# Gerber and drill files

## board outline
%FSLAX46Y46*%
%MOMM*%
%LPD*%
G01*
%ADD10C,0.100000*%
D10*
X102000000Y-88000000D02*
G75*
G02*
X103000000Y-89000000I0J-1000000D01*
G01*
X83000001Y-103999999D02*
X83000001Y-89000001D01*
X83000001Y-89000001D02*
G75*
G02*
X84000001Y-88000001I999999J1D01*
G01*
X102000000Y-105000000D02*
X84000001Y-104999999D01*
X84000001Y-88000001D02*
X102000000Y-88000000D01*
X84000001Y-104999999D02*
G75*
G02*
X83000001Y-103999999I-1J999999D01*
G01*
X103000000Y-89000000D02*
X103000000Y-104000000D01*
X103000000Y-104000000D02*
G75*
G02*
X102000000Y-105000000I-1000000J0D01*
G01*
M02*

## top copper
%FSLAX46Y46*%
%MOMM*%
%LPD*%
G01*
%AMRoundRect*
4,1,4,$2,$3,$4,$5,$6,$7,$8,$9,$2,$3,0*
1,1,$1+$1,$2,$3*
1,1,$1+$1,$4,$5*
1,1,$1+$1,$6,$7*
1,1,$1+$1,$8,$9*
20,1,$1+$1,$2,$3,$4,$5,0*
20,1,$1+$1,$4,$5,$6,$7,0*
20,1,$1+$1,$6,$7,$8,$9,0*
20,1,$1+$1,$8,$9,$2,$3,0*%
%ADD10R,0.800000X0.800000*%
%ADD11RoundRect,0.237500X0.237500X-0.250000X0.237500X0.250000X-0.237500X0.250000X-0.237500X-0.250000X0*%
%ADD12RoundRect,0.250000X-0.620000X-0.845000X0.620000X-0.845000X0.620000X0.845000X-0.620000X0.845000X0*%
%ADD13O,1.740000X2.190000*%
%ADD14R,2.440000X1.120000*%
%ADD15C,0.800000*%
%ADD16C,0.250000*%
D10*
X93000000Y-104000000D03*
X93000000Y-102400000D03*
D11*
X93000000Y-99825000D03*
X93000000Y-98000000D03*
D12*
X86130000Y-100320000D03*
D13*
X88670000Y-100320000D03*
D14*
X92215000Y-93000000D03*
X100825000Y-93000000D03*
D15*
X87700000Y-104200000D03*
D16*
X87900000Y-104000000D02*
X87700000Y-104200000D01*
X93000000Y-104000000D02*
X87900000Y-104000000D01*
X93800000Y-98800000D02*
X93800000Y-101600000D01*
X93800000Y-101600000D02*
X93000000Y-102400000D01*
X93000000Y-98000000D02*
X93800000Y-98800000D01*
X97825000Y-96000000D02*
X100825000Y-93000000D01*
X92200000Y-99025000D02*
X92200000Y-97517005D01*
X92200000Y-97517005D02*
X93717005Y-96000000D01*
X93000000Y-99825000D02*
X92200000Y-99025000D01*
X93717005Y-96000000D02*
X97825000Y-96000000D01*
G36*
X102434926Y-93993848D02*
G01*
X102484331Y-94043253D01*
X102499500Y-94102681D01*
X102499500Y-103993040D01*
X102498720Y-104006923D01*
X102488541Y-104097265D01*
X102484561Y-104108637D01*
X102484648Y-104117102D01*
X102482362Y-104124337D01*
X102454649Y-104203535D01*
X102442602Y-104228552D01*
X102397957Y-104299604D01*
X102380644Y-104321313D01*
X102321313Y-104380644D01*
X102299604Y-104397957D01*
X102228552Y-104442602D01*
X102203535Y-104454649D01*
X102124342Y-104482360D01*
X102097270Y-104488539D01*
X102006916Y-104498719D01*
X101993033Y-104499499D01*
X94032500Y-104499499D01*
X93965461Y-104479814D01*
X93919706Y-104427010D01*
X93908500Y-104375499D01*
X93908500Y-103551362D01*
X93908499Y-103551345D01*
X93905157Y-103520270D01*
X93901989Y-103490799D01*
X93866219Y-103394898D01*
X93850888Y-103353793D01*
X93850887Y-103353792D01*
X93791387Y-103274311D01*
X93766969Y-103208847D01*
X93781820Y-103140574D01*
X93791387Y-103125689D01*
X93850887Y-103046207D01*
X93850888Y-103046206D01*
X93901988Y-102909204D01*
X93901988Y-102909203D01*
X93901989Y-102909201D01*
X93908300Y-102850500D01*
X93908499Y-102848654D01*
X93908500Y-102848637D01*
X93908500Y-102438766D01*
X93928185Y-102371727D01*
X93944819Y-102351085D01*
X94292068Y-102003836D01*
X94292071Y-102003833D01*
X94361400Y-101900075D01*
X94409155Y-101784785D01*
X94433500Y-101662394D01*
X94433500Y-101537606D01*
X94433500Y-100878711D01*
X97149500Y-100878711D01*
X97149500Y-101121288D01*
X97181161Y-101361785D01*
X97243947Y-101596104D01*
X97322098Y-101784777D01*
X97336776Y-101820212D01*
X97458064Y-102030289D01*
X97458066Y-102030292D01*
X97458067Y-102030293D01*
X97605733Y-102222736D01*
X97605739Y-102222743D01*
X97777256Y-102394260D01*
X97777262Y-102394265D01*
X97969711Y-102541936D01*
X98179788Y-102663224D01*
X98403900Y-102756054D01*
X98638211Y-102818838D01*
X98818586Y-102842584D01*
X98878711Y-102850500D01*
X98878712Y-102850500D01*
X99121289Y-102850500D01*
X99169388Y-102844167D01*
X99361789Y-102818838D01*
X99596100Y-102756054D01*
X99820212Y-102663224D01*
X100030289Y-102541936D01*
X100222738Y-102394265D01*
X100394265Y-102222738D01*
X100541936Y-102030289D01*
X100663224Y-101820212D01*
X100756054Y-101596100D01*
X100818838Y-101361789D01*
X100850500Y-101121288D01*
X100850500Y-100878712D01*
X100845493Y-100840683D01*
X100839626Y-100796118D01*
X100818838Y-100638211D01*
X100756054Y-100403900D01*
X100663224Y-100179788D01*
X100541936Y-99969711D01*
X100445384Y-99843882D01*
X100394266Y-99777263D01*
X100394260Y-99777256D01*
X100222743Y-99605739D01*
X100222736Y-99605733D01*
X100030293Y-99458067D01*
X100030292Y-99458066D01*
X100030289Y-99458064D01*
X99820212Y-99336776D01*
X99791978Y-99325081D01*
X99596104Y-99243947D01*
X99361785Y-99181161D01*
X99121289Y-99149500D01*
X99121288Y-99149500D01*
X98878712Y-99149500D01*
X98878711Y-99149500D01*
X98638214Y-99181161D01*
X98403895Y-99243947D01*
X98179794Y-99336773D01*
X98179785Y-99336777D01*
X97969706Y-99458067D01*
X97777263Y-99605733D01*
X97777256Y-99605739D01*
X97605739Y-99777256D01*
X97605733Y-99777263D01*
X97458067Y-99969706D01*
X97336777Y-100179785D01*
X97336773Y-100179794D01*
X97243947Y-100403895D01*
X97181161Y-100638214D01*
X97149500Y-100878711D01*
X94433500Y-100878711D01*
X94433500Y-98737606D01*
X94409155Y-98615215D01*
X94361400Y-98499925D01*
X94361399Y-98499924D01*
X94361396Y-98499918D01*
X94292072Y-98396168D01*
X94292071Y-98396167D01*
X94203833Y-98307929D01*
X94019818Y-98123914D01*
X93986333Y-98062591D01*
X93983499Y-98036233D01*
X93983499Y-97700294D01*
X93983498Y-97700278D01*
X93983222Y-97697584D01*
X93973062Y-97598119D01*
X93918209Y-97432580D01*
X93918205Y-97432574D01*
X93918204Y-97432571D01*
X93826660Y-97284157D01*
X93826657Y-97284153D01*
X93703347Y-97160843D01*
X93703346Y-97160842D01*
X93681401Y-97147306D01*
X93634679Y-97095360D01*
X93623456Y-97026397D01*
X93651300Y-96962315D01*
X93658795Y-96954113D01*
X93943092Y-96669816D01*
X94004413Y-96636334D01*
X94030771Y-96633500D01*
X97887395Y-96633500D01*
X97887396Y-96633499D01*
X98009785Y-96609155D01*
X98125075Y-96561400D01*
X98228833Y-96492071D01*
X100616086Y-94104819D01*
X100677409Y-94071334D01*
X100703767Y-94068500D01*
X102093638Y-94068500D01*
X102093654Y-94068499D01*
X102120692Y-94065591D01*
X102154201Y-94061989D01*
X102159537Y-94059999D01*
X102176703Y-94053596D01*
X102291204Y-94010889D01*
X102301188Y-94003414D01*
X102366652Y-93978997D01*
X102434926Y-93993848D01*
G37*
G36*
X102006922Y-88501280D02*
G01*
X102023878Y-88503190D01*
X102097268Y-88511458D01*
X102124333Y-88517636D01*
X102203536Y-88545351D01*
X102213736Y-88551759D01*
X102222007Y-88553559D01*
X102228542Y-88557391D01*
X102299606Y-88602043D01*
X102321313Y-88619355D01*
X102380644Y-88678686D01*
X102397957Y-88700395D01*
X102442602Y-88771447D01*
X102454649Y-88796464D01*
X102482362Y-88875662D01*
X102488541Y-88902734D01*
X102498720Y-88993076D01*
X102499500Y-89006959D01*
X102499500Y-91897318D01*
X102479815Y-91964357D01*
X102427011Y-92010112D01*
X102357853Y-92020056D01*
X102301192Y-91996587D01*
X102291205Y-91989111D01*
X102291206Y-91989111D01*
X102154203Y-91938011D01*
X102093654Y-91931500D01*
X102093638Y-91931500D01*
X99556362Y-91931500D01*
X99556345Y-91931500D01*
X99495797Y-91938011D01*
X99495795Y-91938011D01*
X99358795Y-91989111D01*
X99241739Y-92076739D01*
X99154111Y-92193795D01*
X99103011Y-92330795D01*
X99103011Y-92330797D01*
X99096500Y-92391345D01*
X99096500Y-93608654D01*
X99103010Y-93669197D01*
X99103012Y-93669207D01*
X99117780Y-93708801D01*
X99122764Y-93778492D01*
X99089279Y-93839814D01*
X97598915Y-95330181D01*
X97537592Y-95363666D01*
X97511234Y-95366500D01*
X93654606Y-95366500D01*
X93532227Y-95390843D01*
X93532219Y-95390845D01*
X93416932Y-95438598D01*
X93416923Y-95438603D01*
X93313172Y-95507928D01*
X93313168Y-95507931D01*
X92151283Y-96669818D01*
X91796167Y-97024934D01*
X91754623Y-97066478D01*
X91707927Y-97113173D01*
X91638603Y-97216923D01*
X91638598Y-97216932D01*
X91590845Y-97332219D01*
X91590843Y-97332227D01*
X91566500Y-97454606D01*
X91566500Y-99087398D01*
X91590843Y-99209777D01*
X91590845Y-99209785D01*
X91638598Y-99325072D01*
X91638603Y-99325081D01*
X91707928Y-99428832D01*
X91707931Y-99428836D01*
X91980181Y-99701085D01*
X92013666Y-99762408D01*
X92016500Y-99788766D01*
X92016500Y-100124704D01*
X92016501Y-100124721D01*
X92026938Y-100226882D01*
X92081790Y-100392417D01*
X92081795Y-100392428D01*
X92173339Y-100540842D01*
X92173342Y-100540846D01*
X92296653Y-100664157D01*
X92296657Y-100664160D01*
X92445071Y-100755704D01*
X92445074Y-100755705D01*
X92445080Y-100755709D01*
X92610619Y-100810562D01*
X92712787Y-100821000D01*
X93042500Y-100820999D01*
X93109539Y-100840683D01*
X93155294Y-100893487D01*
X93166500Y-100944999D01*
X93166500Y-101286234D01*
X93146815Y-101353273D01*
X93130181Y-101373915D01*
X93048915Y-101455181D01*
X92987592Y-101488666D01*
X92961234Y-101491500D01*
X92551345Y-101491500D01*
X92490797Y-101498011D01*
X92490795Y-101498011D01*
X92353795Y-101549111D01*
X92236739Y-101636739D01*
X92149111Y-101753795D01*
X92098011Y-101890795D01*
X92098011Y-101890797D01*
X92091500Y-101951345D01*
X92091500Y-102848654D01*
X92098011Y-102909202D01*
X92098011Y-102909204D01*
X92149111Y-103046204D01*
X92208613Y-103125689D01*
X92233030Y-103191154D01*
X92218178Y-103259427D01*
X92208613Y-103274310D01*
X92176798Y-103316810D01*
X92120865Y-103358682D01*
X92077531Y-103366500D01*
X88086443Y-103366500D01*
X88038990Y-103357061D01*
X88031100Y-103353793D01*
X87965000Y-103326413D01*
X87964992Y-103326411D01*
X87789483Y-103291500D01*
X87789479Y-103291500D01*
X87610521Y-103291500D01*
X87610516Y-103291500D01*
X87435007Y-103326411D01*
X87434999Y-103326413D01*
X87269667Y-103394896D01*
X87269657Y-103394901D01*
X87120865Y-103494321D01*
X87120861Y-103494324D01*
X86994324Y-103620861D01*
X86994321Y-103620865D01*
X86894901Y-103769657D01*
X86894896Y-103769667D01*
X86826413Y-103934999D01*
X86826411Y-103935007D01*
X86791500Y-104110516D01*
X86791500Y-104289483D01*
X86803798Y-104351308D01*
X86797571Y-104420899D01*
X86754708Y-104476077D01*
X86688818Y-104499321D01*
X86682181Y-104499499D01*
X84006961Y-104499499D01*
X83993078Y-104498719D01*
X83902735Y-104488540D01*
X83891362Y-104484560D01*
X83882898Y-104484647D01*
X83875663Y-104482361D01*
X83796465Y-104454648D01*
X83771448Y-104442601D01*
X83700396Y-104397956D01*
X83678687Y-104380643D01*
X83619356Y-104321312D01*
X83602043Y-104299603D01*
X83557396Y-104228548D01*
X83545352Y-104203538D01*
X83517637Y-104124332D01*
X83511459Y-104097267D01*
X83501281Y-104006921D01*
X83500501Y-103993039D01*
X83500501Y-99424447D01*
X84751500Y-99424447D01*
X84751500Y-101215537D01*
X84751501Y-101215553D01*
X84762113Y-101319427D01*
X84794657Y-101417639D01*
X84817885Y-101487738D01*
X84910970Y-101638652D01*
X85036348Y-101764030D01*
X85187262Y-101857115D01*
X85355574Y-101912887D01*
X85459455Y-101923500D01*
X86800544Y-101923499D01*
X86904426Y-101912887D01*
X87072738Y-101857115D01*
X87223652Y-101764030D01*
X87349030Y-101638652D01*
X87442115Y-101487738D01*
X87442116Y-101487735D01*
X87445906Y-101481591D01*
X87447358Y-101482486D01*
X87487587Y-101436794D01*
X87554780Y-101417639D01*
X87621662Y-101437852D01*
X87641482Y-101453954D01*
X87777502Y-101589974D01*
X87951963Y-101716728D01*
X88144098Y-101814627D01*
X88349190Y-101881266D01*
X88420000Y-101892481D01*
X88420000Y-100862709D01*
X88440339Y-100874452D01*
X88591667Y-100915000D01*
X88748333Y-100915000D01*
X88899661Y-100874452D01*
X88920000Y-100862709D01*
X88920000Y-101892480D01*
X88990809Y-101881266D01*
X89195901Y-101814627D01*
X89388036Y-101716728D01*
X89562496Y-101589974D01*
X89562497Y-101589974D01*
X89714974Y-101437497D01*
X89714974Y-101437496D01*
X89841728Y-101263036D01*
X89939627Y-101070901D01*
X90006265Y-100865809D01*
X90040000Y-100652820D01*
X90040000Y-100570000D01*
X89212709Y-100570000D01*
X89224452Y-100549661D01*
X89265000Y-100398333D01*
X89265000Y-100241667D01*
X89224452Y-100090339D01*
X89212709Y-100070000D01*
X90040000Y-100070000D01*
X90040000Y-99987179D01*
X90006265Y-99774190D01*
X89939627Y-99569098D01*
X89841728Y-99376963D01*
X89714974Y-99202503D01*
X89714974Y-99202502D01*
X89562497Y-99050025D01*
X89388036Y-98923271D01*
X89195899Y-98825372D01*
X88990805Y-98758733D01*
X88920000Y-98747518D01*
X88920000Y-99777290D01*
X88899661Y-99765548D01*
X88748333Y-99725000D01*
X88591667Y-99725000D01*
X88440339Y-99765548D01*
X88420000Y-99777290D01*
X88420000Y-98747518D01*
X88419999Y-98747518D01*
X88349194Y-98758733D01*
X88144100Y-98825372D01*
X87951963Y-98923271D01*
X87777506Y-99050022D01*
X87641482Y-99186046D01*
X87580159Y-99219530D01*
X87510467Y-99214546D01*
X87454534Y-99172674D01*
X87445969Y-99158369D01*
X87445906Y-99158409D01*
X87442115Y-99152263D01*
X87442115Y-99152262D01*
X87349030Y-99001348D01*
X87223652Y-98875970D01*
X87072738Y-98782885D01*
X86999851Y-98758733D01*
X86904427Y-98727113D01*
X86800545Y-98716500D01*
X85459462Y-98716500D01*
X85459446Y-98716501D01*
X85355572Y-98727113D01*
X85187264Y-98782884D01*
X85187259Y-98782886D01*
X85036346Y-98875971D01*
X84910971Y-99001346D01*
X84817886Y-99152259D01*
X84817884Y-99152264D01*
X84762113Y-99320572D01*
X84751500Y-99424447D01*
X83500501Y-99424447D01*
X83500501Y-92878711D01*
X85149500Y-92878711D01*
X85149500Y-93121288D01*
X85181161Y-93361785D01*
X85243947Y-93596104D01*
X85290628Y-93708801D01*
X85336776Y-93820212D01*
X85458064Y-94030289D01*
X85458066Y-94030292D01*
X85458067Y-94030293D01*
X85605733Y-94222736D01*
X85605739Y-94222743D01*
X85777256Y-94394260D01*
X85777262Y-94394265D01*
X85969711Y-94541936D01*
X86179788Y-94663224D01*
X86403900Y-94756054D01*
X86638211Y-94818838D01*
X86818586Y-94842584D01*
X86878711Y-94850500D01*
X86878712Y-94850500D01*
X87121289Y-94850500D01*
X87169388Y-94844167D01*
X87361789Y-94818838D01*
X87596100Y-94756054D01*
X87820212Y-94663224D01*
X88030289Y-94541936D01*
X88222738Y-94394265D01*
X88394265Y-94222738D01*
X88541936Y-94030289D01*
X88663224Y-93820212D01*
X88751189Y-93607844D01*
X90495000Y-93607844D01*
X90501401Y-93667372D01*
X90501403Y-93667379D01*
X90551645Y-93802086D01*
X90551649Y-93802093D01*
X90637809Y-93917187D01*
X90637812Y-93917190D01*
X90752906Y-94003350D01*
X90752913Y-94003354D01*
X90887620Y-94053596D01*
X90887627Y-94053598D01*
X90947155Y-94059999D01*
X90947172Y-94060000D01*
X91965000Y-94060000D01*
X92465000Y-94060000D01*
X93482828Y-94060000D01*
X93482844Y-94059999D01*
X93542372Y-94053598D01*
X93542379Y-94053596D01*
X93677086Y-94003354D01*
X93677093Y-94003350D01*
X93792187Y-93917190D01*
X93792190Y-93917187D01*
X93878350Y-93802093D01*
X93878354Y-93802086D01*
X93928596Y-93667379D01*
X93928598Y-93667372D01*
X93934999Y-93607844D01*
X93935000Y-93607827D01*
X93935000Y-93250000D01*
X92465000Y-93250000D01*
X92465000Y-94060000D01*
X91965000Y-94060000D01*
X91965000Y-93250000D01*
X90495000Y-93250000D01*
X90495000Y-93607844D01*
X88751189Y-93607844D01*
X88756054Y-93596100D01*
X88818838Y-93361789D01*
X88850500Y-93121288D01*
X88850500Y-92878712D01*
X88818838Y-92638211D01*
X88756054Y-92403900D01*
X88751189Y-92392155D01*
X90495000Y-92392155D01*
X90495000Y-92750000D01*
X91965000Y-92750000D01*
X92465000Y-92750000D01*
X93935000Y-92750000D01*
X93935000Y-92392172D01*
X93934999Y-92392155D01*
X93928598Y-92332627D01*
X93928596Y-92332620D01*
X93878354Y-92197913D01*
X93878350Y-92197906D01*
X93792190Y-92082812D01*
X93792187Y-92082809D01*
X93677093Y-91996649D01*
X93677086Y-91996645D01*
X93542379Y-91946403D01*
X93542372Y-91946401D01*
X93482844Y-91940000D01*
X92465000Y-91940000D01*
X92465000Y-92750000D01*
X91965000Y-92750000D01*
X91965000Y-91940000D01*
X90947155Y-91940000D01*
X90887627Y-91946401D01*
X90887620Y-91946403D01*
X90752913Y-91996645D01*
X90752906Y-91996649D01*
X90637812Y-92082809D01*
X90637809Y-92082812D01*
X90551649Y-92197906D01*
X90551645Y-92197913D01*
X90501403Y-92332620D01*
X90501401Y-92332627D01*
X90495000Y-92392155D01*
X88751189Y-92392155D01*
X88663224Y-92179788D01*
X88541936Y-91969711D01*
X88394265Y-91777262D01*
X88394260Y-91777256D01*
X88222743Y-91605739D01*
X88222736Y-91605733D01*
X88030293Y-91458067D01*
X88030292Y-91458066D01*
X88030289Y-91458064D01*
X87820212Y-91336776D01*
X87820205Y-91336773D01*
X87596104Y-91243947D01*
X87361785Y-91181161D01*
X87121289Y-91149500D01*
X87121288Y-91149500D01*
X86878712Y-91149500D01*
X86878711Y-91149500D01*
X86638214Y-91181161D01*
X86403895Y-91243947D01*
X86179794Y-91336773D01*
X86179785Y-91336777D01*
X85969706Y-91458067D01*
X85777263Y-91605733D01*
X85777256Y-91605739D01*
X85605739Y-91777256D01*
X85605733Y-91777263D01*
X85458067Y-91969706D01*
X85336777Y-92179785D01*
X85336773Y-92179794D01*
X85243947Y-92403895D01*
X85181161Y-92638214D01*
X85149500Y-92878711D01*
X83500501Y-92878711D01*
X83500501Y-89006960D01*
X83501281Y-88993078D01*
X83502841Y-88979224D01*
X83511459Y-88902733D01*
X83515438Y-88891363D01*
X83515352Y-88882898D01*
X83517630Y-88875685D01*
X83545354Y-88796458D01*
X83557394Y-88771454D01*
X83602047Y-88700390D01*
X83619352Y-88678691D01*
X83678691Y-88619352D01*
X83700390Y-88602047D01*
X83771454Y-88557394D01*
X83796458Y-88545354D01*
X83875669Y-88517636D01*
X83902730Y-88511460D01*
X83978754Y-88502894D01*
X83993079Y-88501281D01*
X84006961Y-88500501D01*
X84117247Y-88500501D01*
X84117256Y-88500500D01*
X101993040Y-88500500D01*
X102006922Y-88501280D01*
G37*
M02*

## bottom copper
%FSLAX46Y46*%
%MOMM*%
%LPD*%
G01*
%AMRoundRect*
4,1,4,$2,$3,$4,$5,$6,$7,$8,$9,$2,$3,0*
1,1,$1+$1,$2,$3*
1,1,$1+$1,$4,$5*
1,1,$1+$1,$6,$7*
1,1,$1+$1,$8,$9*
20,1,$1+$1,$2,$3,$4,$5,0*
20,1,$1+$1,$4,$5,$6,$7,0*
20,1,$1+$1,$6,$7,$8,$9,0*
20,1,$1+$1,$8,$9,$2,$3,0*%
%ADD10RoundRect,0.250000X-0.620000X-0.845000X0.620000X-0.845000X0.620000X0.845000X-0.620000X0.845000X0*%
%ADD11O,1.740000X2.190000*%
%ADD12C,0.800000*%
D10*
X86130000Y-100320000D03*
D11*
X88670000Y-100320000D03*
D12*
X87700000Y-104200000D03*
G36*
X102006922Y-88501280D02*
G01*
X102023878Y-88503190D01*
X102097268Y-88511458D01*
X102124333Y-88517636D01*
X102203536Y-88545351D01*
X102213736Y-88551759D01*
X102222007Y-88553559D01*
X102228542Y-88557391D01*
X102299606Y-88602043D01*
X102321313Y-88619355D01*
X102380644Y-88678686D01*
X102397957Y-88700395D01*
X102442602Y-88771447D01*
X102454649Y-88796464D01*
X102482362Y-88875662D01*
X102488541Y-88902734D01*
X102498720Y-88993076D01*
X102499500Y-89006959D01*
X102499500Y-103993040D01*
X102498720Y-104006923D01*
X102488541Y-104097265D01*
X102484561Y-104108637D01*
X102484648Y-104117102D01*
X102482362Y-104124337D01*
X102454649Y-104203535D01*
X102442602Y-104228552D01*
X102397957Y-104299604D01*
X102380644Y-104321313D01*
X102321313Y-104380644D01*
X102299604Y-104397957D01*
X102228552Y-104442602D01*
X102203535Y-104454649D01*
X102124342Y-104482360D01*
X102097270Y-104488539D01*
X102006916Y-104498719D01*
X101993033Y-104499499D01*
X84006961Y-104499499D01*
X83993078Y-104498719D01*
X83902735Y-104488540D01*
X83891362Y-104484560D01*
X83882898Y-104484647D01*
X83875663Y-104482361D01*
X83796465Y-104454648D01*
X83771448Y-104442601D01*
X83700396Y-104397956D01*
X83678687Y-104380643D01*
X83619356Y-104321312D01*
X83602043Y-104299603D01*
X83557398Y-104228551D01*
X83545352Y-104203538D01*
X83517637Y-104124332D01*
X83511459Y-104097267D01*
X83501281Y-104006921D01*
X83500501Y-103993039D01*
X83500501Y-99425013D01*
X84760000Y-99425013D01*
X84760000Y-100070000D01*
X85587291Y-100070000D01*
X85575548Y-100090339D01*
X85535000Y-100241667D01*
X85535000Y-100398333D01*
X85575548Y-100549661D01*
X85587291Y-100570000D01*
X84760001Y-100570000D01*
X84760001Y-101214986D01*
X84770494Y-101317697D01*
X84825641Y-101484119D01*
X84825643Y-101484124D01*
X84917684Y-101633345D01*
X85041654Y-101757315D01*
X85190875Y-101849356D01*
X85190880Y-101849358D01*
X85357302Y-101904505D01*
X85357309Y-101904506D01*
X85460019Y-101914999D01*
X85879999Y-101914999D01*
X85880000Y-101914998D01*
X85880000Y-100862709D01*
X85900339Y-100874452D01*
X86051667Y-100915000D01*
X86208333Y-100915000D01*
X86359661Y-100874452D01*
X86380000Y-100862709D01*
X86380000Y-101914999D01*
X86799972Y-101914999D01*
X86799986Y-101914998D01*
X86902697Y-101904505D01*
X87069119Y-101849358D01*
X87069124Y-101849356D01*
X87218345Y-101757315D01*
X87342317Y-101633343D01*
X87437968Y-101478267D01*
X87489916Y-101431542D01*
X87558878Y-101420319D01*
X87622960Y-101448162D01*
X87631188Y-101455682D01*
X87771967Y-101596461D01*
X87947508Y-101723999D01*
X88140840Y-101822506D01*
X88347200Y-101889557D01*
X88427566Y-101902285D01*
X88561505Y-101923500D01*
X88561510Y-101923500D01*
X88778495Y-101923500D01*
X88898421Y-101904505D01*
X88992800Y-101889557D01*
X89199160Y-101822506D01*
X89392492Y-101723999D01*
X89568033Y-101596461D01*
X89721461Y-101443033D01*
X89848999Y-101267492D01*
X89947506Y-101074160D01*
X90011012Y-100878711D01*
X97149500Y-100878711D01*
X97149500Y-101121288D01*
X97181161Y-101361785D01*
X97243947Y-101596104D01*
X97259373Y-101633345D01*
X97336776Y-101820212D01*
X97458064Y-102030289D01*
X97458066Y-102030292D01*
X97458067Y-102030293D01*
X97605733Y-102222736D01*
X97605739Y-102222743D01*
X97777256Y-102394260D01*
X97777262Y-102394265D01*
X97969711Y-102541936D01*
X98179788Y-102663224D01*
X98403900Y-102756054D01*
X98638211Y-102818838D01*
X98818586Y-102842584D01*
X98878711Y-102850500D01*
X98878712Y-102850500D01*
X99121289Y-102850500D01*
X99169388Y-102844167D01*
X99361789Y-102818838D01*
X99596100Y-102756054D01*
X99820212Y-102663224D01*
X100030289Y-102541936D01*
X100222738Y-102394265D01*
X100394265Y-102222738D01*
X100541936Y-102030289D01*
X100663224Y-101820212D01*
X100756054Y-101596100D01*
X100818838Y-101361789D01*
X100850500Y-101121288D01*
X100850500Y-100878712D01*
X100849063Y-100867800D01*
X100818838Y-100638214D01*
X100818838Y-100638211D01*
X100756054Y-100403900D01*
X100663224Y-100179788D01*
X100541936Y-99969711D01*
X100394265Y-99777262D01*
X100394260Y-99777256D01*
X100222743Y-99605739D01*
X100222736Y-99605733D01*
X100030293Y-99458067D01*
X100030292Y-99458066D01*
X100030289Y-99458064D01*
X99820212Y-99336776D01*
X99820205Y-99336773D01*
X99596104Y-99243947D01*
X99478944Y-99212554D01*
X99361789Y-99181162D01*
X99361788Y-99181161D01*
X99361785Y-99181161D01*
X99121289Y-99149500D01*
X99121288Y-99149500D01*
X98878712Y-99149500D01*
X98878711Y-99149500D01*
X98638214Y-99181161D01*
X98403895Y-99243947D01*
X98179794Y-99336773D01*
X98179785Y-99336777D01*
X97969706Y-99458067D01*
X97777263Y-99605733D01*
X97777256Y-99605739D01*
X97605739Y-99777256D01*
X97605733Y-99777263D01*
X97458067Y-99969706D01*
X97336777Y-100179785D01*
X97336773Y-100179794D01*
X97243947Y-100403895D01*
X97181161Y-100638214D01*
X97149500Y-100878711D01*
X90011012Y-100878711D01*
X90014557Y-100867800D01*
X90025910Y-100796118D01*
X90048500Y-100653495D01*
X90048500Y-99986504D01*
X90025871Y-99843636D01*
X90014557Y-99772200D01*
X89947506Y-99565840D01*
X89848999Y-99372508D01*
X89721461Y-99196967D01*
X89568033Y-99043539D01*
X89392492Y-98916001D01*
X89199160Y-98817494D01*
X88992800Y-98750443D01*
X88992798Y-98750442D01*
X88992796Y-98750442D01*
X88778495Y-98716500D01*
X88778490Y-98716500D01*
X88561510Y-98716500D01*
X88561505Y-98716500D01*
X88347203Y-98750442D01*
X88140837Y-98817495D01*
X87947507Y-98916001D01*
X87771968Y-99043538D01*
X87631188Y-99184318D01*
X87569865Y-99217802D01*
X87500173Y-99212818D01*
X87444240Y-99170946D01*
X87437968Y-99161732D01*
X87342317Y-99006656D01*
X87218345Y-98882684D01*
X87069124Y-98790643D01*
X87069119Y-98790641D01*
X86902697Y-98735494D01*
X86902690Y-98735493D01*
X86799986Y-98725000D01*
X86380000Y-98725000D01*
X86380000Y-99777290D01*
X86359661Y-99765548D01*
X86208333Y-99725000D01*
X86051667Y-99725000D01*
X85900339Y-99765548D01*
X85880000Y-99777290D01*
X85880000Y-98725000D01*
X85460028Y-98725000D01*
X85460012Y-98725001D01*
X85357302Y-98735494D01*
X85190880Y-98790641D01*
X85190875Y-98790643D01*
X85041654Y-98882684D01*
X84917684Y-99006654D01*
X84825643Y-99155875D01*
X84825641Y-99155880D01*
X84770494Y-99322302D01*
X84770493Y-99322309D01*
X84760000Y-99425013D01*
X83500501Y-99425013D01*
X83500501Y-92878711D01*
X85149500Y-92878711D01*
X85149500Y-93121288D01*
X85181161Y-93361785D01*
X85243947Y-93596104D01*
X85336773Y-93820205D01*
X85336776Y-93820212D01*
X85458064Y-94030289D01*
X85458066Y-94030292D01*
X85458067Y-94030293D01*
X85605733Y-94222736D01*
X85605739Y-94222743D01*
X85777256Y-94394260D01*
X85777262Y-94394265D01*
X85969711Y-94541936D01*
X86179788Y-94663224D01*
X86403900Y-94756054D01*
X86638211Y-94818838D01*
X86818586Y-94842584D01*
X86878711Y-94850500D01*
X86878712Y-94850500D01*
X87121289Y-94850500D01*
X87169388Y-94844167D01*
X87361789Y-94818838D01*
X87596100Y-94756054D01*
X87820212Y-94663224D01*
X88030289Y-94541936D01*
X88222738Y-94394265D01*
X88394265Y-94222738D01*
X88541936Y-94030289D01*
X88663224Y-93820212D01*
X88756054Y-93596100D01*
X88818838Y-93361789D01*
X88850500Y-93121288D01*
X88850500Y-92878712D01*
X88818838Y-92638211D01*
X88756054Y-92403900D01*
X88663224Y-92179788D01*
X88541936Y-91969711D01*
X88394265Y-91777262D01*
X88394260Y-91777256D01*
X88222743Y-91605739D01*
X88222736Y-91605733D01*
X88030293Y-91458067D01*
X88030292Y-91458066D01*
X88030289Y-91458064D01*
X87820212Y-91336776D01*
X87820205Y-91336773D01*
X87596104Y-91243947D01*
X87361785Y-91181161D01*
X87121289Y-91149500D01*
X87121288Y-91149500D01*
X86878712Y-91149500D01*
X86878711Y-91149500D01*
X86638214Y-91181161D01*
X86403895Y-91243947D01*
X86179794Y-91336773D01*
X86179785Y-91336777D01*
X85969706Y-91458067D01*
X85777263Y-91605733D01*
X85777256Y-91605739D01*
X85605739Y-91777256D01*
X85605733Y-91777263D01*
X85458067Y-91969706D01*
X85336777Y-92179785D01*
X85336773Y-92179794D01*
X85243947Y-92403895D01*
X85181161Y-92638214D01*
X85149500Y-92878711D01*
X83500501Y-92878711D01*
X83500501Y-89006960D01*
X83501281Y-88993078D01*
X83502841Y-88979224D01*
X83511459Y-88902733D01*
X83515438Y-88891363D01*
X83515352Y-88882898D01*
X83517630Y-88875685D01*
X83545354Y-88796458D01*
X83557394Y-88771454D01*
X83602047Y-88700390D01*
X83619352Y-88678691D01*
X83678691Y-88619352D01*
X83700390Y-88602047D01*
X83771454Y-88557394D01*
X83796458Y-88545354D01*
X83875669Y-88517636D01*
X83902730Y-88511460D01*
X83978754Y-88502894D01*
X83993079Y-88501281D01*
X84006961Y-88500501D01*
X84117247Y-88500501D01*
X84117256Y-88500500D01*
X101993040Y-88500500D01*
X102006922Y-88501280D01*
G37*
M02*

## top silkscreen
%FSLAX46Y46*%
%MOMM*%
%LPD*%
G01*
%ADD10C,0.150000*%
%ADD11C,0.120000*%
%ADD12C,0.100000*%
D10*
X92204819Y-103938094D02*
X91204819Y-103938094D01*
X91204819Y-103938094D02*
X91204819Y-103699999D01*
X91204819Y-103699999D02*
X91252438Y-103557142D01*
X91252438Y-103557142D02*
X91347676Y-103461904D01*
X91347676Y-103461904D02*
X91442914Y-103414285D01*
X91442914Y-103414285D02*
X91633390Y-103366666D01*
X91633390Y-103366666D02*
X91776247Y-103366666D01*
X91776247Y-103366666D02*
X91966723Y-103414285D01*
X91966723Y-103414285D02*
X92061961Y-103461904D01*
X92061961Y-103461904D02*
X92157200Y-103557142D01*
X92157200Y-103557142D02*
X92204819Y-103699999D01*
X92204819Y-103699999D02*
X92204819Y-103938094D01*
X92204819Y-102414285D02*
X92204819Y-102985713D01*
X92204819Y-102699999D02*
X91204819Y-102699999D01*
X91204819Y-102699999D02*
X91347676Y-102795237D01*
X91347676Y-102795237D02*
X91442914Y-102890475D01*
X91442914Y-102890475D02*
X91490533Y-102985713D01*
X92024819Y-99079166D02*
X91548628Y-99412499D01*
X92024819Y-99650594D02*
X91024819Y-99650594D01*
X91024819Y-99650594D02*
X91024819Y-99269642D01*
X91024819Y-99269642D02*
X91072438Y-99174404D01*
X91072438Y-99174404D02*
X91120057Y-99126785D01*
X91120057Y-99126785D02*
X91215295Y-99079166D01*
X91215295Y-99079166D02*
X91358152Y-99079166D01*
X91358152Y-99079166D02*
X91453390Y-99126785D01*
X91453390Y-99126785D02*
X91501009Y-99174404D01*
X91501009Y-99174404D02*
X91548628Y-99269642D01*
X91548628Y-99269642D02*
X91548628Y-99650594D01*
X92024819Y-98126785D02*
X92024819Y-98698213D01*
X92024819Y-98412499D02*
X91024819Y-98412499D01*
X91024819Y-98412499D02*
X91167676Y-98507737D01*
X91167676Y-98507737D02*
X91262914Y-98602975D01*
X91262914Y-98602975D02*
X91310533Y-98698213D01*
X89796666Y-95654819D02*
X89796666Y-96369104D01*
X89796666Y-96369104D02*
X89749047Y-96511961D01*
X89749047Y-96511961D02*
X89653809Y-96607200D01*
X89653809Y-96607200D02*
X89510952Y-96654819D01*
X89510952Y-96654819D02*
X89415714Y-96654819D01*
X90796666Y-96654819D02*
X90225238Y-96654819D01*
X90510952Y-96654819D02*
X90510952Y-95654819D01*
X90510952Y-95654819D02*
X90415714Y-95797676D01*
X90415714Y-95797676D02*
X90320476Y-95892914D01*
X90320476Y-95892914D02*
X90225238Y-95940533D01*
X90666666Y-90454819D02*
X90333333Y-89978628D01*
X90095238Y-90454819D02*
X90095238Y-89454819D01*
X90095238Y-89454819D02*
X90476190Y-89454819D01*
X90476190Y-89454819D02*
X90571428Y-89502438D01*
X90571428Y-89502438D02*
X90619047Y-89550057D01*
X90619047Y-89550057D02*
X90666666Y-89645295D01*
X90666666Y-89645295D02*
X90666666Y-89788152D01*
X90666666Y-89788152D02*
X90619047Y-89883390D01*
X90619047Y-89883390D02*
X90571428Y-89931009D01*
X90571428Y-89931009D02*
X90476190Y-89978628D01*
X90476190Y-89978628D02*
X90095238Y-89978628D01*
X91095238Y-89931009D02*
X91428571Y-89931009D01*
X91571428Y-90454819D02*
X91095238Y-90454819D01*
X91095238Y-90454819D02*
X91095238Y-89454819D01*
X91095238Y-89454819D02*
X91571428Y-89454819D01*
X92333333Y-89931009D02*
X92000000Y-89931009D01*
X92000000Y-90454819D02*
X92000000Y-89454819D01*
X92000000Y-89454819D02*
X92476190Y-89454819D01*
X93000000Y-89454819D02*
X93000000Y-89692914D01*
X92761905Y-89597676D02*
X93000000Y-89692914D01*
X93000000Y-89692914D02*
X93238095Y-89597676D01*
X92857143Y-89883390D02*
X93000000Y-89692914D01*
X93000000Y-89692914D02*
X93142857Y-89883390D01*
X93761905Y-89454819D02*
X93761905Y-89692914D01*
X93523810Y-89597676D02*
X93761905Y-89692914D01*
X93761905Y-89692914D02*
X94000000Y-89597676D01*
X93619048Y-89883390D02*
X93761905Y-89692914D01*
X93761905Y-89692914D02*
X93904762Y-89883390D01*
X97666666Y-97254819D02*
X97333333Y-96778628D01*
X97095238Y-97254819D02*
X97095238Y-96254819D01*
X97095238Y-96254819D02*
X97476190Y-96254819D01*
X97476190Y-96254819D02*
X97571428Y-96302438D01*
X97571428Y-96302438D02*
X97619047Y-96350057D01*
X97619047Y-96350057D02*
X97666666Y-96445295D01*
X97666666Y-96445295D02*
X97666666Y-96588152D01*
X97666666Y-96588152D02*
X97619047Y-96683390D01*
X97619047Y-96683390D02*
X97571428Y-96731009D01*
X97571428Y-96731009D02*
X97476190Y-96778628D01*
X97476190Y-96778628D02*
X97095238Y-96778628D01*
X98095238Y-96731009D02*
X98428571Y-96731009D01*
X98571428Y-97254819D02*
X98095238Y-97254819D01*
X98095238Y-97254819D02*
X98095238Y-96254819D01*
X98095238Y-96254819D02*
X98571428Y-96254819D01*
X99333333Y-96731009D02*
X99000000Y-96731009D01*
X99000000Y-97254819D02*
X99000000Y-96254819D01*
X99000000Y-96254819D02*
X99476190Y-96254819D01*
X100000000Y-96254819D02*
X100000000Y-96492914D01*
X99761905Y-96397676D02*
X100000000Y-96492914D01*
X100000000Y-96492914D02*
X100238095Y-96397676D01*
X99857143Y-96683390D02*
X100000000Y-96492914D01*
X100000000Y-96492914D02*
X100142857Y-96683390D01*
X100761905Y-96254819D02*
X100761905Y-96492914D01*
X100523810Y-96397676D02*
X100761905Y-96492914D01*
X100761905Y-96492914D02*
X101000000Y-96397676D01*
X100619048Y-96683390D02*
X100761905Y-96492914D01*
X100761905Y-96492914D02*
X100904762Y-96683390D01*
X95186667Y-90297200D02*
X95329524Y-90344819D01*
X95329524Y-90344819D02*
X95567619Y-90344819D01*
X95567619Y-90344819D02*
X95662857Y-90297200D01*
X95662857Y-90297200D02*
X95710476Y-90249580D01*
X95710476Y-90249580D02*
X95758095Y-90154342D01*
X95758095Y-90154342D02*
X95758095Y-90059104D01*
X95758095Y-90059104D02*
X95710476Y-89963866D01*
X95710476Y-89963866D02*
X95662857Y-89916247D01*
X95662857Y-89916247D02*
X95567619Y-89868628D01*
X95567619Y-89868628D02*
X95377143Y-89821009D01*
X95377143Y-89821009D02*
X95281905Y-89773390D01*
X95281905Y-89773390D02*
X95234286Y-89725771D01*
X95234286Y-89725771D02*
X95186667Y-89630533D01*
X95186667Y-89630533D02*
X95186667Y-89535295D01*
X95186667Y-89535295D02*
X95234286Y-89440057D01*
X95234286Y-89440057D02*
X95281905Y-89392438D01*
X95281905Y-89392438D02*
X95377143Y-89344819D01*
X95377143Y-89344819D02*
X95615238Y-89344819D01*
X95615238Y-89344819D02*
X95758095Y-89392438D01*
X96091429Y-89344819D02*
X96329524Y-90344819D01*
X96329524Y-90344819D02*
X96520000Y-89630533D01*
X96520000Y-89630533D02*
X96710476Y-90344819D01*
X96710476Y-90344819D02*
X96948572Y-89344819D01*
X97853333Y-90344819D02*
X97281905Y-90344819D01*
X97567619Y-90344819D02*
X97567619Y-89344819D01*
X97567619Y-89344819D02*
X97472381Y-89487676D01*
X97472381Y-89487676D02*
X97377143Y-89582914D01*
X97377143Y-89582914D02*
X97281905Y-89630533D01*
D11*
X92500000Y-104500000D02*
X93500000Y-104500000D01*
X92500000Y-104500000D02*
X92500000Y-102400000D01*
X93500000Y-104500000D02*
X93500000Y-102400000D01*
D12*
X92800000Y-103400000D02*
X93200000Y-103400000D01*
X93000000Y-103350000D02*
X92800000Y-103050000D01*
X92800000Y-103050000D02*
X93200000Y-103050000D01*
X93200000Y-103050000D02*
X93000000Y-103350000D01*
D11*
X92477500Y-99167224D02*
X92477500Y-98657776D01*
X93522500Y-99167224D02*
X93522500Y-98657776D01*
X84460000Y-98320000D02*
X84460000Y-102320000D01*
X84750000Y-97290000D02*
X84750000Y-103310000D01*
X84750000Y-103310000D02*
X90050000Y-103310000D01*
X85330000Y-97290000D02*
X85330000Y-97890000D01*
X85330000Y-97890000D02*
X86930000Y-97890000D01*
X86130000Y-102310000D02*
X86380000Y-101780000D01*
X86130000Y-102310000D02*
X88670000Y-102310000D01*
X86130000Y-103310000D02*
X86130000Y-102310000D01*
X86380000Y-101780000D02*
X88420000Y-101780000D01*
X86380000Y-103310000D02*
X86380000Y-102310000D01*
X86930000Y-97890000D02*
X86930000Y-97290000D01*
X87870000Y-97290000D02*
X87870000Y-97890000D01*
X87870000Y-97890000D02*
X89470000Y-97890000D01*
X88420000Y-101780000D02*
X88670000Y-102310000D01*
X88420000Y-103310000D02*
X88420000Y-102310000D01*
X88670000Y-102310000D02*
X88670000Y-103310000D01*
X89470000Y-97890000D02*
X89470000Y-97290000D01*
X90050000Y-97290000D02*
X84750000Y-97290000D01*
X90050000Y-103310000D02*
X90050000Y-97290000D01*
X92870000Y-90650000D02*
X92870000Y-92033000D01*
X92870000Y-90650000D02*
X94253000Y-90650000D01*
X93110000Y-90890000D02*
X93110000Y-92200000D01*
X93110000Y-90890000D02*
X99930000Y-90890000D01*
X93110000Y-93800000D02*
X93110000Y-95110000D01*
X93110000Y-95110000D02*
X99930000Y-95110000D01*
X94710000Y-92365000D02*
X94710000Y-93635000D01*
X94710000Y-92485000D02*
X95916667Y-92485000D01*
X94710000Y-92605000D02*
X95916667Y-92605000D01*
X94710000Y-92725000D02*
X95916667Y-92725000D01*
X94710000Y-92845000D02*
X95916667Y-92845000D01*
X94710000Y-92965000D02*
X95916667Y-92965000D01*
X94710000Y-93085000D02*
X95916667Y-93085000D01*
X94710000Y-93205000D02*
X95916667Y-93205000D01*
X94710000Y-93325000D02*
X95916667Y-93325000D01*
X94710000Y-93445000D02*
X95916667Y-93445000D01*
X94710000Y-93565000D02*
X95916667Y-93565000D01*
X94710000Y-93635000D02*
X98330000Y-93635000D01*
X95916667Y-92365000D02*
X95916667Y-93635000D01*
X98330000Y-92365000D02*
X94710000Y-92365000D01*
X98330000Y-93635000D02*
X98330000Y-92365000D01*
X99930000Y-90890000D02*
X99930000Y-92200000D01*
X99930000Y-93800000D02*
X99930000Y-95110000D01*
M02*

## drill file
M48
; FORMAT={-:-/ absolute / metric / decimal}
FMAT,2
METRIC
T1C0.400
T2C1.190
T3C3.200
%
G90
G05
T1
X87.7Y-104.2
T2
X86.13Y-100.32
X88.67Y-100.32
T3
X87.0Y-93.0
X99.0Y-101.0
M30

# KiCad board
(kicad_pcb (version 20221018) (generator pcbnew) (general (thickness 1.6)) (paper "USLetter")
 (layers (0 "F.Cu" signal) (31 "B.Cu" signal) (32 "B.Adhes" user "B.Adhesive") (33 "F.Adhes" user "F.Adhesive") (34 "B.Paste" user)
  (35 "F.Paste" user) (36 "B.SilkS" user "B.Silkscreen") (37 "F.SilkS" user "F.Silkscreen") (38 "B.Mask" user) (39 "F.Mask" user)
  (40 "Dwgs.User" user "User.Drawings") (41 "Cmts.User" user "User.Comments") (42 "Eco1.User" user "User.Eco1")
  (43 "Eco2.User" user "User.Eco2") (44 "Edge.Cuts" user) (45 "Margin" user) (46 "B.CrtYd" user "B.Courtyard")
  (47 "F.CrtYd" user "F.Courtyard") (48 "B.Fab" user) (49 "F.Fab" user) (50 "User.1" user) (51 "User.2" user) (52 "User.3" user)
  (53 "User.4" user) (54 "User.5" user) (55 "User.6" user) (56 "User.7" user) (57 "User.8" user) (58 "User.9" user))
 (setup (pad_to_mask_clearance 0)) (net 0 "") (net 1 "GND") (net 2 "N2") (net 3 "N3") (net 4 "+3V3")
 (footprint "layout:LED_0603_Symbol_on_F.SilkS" (layer "F.Cu") (at 93 103.2 90)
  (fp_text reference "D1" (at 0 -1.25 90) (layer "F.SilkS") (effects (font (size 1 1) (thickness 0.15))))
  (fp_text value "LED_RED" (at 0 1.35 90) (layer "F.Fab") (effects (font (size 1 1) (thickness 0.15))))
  (fp_line (start -1.3 -0.5) (end -1.3 0.5) (stroke (width 0.12) (type solid)) (layer "F.SilkS"))
  (fp_line (start -1.3 -0.5) (end 0.8 -0.5) (stroke (width 0.12) (type solid)) (layer "F.SilkS"))
  (fp_line (start -1.3 0.5) (end 0.8 0.5) (stroke (width 0.12) (type solid)) (layer "F.SilkS"))
  (fp_line (start -0.2 -0.2) (end -0.2 0.2) (stroke (width 0.1) (type solid)) (layer "F.SilkS"))
  (fp_line (start -0.15 0) (end 0.15 -0.2) (stroke (width 0.1) (type solid)) (layer "F.SilkS"))
  (fp_line (start 0.15 -0.2) (end 0.15 0.2) (stroke (width 0.1) (type solid)) (layer "F.SilkS"))
  (fp_line (start 0.15 0.2) (end -0.15 0) (stroke (width 0.1) (type solid)) (layer "F.SilkS"))
  (pad "1" smd rect (at -0.8 0 270) (size 0.8 0.8) (layers "F.Cu" "F.Paste" "F.Mask") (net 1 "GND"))
  (pad "2" smd rect (at 0.8 0 270) (size 0.8 0.8) (layers "F.Cu" "F.Paste" "F.Mask") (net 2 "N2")))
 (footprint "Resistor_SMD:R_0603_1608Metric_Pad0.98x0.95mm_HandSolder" (layer "F.Cu") (at 93 98.9125 90)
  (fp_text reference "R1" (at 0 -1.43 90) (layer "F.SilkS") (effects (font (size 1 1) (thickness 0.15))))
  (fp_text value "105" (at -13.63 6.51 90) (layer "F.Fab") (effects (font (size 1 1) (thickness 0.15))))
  (fp_line (start -0.254724 -0.5225) (end 0.254724 -0.5225) (stroke (width 0.12) (type solid)) (layer "F.SilkS"))
  (fp_line (start -0.254724 0.5225) (end 0.254724 0.5225) (stroke (width 0.12) (type solid)) (layer "F.SilkS"))
  (pad "1" smd roundrect (at -0.9125 0 90) (size 0.975 0.95) (layers "F.Cu" "F.Paste" "F.Mask") (roundrect_rratio 0.25) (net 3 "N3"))
  (pad "2" smd roundrect (at 0.9125 0 90) (size 0.975 0.95) (layers "F.Cu" "F.Paste" "F.Mask") (roundrect_rratio 0.25) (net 2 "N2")))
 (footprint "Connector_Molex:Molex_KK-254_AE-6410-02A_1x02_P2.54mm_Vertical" (layer "F.Cu") (at 86.13 100.32)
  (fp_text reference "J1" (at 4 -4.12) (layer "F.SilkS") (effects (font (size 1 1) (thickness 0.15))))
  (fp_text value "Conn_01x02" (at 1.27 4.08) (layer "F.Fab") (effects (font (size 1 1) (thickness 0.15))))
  (fp_line (start -1.67 -2) (end -1.67 2) (stroke (width 0.12) (type solid)) (layer "F.SilkS"))
  (fp_line (start -1.38 -3.03) (end -1.38 2.99) (stroke (width 0.12) (type solid)) (layer "F.SilkS"))
  (fp_line (start -1.38 2.99) (end 3.92 2.99) (stroke (width 0.12) (type solid)) (layer "F.SilkS"))
  (fp_line (start -0.8 -3.03) (end -0.8 -2.43) (stroke (width 0.12) (type solid)) (layer "F.SilkS"))
  (fp_line (start -0.8 -2.43) (end 0.8 -2.43) (stroke (width 0.12) (type solid)) (layer "F.SilkS"))
  (fp_line (start 0 1.99) (end 0.25 1.46) (stroke (width 0.12) (type solid)) (layer "F.SilkS"))
  (fp_line (start 0 1.99) (end 2.54 1.99) (stroke (width 0.12) (type solid)) (layer "F.SilkS"))
  (fp_line (start 0 2.99) (end 0 1.99) (stroke (width 0.12) (type solid)) (layer "F.SilkS"))
  (fp_line (start 0.25 1.46) (end 2.29 1.46) (stroke (width 0.12) (type solid)) (layer "F.SilkS"))
  (fp_line (start 0.25 2.99) (end 0.25 1.99) (stroke (width 0.12) (type solid)) (layer "F.SilkS"))
  (fp_line (start 0.8 -2.43) (end 0.8 -3.03) (stroke (width 0.12) (type solid)) (layer "F.SilkS"))
  (fp_line (start 1.74 -3.03) (end 1.74 -2.43) (stroke (width 0.12) (type solid)) (layer "F.SilkS"))
  (fp_line (start 1.74 -2.43) (end 3.34 -2.43) (stroke (width 0.12) (type solid)) (layer "F.SilkS"))
  (fp_line (start 2.29 1.46) (end 2.54 1.99) (stroke (width 0.12) (type solid)) (layer "F.SilkS"))
  (fp_line (start 2.29 2.99) (end 2.29 1.99) (stroke (width 0.12) (type solid)) (layer "F.SilkS"))
  (fp_line (start 2.54 1.99) (end 2.54 2.99) (stroke (width 0.12) (type solid)) (layer "F.SilkS"))
  (fp_line (start 3.34 -2.43) (end 3.34 -3.03) (stroke (width 0.12) (type solid)) (layer "F.SilkS"))
  (fp_line (start 3.92 -3.03) (end -1.38 -3.03) (stroke (width 0.12) (type solid)) (layer "F.SilkS"))
  (fp_line (start 3.92 2.99) (end 3.92 -3.03) (stroke (width 0.12) (type solid)) (layer "F.SilkS"))
  (pad "1" thru_hole roundrect (at 0 0) (size 1.74 2.19) (drill 1.19) (layers "*.Cu" "*.Mask") (roundrect_rratio 0.143678) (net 1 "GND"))
  (pad "2" thru_hole oval (at 2.54 0) (size 1.74 2.19) (drill 1.19) (layers "*.Cu" "*.Mask") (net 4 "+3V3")))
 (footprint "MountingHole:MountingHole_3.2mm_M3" (layer "F.Cu") (at 87 93)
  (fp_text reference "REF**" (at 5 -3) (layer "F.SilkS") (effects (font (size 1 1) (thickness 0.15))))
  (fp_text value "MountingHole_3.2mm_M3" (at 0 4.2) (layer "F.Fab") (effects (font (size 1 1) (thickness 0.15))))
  (pad "" np_thru_hole circle (at 0 0) (size 3.2 3.2) (drill 3.2) (layers "*.Cu" "*.Mask")))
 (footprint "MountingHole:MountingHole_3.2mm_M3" (layer "F.Cu") (at 99 101)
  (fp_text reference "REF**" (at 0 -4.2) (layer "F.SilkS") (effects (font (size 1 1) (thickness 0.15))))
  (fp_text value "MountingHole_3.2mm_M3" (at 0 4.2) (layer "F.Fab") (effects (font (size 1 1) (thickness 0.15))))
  (pad "" np_thru_hole circle (at 0 0) (size 3.2 3.2) (drill 3.2) (layers "F&B.Cu" "*.Mask")))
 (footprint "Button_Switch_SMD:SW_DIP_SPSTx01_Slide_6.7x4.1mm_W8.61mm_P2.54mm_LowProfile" (layer "F.Cu") (at 96.52 93)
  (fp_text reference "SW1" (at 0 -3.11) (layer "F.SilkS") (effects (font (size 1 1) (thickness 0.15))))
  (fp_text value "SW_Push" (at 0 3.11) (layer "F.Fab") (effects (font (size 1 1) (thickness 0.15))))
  (fp_line (start -3.65 -2.35) (end -3.65 -0.967) (stroke (width 0.12) (type solid)) (layer "F.SilkS"))
  (fp_line (start -3.65 -2.35) (end -2.267 -2.35) (stroke (width 0.12) (type solid)) (layer "F.SilkS"))
  (fp_line (start -3.41 -2.11) (end -3.41 -0.8) (stroke (width 0.12) (type solid)) (layer "F.SilkS"))
  (fp_line (start -3.41 -2.11) (end 3.41 -2.11) (stroke (width 0.12) (type solid)) (layer "F.SilkS"))
  (fp_line (start -3.41 0.8) (end -3.41 2.11) (stroke (width 0.12) (type solid)) (layer "F.SilkS"))
  (fp_line (start -3.41 2.11) (end 3.41 2.11) (stroke (width 0.12) (type solid)) (layer "F.SilkS"))
  (fp_line (start -1.81 -0.635) (end -1.81 0.635) (stroke (width 0.12) (type solid)) (layer "F.SilkS"))
  (fp_line (start -1.81 -0.515) (end -0.603333 -0.515) (stroke (width 0.12) (type solid)) (layer "F.SilkS"))
  (fp_line (start -1.81 -0.395) (end -0.603333 -0.395) (stroke (width 0.12) (type solid)) (layer "F.SilkS"))
  (fp_line (start -1.81 -0.275) (end -0.603333 -0.275) (stroke (width 0.12) (type solid)) (layer "F.SilkS"))
  (fp_line (start -1.81 -0.155) (end -0.603333 -0.155) (stroke (width 0.12) (type solid)) (layer "F.SilkS"))
  (fp_line (start -1.81 -0.035) (end -0.603333 -0.035) (stroke (width 0.12) (type solid)) (layer "F.SilkS"))
  (fp_line (start -1.81 0.085) (end -0.603333 0.085) (stroke (width 0.12) (type solid)) (layer "F.SilkS"))
  (fp_line (start -1.81 0.205) (end -0.603333 0.205) (stroke (width 0.12) (type solid)) (layer "F.SilkS"))
  (fp_line (start -1.81 0.325) (end -0.603333 0.325) (stroke (width 0.12) (type solid)) (layer "F.SilkS"))
  (fp_line (start -1.81 0.445) (end -0.603333 0.445) (stroke (width 0.12) (type solid)) (layer "F.SilkS"))
  (fp_line (start -1.81 0.565) (end -0.603333 0.565) (stroke (width 0.12) (type solid)) (layer "F.SilkS"))
  (fp_line (start -1.81 0.635) (end 1.81 0.635) (stroke (width 0.12) (type solid)) (layer "F.SilkS"))
  (fp_line (start -0.603333 -0.635) (end -0.603333 0.635) (stroke (width 0.12) (type solid)) (layer "F.SilkS"))
  (fp_line (start 1.81 -0.635) (end -1.81 -0.635) (stroke (width 0.12) (type solid)) (layer "F.SilkS"))
  (fp_line (start 1.81 0.635) (end 1.81 -0.635) (stroke (width 0.12) (type solid)) (layer "F.SilkS"))
  (fp_line (start 3.41 -2.11) (end 3.41 -0.8) (stroke (width 0.12) (type solid)) (layer "F.SilkS"))
  (fp_line (start 3.41 0.8) (end 3.41 2.11) (stroke (width 0.12) (type solid)) (layer "F.SilkS"))
  (pad "1" smd rect (at -4.305 0) (size 2.44 1.12) (layers "F.Cu" "F.Paste" "F.Mask") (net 4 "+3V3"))
  (pad "2" smd rect (at 4.305 0) (size 2.44 1.12) (layers "F.Cu" "F.Paste" "F.Mask") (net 3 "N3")))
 (gr_arc (start 102 88) (mid 102.707107 88.292893) (end 103 89) (stroke (width 0.1) (type default)) (layer "Edge.Cuts"))
 (gr_line (start 83.000001 103.999999) (end 83.000001 89.000001) (stroke (width 0.1) (type default)) (layer "Edge.Cuts"))
 (gr_arc (start 83.000001 89.000001) (mid 83.292894 88.292894) (end 84.000001 88.000001) (stroke (width 0.1) (type default))
  (layer "Edge.Cuts"))
 (gr_line (start 102 105) (end 84.000001 104.999999) (stroke (width 0.1) (type default)) (layer "Edge.Cuts"))
 (gr_line (start 84.000001 88.000001) (end 102 88) (stroke (width 0.1) (type default)) (layer "Edge.Cuts"))
 (gr_arc (start 84.000001 104.999999) (mid 83.292894 104.707106) (end 83.000001 103.999999) (stroke (width 0.1) (type default))
  (layer "Edge.Cuts"))
 (gr_line (start 103 89) (end 103 104) (stroke (width 0.1) (type default)) (layer "Edge.Cuts"))
 (gr_arc (start 103 104) (mid 102.707107 104.707107) (end 102 105) (stroke (width 0.1) (type default)) (layer "Edge.Cuts"))
 (segment (start 87.9 104) (end 87.7 104.2) (width 0.25) (layer "F.Cu") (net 1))
 (segment (start 93 104) (end 87.9 104) (width 0.25) (layer "F.Cu") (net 1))
 (via (at 87.7 104.2) (size 0.8) (drill 0.4) (layers "F.Cu" "B.Cu") (free) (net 1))
 (segment (start 93.8 98.8) (end 93.8 101.6) (width 0.25) (layer "F.Cu") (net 2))
 (segment (start 93.8 101.6) (end 93 102.4) (width 0.25) (layer "F.Cu") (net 2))
 (segment (start 93 98) (end 93.8 98.8) (width 0.25) (layer "F.Cu") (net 2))
 (segment (start 97.825 96) (end 100.825 93) (width 0.25) (layer "F.Cu") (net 3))
 (segment (start 92.2 99.025) (end 92.2 97.517005) (width 0.25) (layer "F.Cu") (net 3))
 (segment (start 92.2 97.517005) (end 93.717005 96) (width 0.25) (layer "F.Cu") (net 3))
 (segment (start 93 99.825) (end 92.2 99.025) (width 0.25) (layer "F.Cu") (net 3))
 (segment (start 93.717005 96) (end 97.825 96) (width 0.25) (layer "F.Cu") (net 3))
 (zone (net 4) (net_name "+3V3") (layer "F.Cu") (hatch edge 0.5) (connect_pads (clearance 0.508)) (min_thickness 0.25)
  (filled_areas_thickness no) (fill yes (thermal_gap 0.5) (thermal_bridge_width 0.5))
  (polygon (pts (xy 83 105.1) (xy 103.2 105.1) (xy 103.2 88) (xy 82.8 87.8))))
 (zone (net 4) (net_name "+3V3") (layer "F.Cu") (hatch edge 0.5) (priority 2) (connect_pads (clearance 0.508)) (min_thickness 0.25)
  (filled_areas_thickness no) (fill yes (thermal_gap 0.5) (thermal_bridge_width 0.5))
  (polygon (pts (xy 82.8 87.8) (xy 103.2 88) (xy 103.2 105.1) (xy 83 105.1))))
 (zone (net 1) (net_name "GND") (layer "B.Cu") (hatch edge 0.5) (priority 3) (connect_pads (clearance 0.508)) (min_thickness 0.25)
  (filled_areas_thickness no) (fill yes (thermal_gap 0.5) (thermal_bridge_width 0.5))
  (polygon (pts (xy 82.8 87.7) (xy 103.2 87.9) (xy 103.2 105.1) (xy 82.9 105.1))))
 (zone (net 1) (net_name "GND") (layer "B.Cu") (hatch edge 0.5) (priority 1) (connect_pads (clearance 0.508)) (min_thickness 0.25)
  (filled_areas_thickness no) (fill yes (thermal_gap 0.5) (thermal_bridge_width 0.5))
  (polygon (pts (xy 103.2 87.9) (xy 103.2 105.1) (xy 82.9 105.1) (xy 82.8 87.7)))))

